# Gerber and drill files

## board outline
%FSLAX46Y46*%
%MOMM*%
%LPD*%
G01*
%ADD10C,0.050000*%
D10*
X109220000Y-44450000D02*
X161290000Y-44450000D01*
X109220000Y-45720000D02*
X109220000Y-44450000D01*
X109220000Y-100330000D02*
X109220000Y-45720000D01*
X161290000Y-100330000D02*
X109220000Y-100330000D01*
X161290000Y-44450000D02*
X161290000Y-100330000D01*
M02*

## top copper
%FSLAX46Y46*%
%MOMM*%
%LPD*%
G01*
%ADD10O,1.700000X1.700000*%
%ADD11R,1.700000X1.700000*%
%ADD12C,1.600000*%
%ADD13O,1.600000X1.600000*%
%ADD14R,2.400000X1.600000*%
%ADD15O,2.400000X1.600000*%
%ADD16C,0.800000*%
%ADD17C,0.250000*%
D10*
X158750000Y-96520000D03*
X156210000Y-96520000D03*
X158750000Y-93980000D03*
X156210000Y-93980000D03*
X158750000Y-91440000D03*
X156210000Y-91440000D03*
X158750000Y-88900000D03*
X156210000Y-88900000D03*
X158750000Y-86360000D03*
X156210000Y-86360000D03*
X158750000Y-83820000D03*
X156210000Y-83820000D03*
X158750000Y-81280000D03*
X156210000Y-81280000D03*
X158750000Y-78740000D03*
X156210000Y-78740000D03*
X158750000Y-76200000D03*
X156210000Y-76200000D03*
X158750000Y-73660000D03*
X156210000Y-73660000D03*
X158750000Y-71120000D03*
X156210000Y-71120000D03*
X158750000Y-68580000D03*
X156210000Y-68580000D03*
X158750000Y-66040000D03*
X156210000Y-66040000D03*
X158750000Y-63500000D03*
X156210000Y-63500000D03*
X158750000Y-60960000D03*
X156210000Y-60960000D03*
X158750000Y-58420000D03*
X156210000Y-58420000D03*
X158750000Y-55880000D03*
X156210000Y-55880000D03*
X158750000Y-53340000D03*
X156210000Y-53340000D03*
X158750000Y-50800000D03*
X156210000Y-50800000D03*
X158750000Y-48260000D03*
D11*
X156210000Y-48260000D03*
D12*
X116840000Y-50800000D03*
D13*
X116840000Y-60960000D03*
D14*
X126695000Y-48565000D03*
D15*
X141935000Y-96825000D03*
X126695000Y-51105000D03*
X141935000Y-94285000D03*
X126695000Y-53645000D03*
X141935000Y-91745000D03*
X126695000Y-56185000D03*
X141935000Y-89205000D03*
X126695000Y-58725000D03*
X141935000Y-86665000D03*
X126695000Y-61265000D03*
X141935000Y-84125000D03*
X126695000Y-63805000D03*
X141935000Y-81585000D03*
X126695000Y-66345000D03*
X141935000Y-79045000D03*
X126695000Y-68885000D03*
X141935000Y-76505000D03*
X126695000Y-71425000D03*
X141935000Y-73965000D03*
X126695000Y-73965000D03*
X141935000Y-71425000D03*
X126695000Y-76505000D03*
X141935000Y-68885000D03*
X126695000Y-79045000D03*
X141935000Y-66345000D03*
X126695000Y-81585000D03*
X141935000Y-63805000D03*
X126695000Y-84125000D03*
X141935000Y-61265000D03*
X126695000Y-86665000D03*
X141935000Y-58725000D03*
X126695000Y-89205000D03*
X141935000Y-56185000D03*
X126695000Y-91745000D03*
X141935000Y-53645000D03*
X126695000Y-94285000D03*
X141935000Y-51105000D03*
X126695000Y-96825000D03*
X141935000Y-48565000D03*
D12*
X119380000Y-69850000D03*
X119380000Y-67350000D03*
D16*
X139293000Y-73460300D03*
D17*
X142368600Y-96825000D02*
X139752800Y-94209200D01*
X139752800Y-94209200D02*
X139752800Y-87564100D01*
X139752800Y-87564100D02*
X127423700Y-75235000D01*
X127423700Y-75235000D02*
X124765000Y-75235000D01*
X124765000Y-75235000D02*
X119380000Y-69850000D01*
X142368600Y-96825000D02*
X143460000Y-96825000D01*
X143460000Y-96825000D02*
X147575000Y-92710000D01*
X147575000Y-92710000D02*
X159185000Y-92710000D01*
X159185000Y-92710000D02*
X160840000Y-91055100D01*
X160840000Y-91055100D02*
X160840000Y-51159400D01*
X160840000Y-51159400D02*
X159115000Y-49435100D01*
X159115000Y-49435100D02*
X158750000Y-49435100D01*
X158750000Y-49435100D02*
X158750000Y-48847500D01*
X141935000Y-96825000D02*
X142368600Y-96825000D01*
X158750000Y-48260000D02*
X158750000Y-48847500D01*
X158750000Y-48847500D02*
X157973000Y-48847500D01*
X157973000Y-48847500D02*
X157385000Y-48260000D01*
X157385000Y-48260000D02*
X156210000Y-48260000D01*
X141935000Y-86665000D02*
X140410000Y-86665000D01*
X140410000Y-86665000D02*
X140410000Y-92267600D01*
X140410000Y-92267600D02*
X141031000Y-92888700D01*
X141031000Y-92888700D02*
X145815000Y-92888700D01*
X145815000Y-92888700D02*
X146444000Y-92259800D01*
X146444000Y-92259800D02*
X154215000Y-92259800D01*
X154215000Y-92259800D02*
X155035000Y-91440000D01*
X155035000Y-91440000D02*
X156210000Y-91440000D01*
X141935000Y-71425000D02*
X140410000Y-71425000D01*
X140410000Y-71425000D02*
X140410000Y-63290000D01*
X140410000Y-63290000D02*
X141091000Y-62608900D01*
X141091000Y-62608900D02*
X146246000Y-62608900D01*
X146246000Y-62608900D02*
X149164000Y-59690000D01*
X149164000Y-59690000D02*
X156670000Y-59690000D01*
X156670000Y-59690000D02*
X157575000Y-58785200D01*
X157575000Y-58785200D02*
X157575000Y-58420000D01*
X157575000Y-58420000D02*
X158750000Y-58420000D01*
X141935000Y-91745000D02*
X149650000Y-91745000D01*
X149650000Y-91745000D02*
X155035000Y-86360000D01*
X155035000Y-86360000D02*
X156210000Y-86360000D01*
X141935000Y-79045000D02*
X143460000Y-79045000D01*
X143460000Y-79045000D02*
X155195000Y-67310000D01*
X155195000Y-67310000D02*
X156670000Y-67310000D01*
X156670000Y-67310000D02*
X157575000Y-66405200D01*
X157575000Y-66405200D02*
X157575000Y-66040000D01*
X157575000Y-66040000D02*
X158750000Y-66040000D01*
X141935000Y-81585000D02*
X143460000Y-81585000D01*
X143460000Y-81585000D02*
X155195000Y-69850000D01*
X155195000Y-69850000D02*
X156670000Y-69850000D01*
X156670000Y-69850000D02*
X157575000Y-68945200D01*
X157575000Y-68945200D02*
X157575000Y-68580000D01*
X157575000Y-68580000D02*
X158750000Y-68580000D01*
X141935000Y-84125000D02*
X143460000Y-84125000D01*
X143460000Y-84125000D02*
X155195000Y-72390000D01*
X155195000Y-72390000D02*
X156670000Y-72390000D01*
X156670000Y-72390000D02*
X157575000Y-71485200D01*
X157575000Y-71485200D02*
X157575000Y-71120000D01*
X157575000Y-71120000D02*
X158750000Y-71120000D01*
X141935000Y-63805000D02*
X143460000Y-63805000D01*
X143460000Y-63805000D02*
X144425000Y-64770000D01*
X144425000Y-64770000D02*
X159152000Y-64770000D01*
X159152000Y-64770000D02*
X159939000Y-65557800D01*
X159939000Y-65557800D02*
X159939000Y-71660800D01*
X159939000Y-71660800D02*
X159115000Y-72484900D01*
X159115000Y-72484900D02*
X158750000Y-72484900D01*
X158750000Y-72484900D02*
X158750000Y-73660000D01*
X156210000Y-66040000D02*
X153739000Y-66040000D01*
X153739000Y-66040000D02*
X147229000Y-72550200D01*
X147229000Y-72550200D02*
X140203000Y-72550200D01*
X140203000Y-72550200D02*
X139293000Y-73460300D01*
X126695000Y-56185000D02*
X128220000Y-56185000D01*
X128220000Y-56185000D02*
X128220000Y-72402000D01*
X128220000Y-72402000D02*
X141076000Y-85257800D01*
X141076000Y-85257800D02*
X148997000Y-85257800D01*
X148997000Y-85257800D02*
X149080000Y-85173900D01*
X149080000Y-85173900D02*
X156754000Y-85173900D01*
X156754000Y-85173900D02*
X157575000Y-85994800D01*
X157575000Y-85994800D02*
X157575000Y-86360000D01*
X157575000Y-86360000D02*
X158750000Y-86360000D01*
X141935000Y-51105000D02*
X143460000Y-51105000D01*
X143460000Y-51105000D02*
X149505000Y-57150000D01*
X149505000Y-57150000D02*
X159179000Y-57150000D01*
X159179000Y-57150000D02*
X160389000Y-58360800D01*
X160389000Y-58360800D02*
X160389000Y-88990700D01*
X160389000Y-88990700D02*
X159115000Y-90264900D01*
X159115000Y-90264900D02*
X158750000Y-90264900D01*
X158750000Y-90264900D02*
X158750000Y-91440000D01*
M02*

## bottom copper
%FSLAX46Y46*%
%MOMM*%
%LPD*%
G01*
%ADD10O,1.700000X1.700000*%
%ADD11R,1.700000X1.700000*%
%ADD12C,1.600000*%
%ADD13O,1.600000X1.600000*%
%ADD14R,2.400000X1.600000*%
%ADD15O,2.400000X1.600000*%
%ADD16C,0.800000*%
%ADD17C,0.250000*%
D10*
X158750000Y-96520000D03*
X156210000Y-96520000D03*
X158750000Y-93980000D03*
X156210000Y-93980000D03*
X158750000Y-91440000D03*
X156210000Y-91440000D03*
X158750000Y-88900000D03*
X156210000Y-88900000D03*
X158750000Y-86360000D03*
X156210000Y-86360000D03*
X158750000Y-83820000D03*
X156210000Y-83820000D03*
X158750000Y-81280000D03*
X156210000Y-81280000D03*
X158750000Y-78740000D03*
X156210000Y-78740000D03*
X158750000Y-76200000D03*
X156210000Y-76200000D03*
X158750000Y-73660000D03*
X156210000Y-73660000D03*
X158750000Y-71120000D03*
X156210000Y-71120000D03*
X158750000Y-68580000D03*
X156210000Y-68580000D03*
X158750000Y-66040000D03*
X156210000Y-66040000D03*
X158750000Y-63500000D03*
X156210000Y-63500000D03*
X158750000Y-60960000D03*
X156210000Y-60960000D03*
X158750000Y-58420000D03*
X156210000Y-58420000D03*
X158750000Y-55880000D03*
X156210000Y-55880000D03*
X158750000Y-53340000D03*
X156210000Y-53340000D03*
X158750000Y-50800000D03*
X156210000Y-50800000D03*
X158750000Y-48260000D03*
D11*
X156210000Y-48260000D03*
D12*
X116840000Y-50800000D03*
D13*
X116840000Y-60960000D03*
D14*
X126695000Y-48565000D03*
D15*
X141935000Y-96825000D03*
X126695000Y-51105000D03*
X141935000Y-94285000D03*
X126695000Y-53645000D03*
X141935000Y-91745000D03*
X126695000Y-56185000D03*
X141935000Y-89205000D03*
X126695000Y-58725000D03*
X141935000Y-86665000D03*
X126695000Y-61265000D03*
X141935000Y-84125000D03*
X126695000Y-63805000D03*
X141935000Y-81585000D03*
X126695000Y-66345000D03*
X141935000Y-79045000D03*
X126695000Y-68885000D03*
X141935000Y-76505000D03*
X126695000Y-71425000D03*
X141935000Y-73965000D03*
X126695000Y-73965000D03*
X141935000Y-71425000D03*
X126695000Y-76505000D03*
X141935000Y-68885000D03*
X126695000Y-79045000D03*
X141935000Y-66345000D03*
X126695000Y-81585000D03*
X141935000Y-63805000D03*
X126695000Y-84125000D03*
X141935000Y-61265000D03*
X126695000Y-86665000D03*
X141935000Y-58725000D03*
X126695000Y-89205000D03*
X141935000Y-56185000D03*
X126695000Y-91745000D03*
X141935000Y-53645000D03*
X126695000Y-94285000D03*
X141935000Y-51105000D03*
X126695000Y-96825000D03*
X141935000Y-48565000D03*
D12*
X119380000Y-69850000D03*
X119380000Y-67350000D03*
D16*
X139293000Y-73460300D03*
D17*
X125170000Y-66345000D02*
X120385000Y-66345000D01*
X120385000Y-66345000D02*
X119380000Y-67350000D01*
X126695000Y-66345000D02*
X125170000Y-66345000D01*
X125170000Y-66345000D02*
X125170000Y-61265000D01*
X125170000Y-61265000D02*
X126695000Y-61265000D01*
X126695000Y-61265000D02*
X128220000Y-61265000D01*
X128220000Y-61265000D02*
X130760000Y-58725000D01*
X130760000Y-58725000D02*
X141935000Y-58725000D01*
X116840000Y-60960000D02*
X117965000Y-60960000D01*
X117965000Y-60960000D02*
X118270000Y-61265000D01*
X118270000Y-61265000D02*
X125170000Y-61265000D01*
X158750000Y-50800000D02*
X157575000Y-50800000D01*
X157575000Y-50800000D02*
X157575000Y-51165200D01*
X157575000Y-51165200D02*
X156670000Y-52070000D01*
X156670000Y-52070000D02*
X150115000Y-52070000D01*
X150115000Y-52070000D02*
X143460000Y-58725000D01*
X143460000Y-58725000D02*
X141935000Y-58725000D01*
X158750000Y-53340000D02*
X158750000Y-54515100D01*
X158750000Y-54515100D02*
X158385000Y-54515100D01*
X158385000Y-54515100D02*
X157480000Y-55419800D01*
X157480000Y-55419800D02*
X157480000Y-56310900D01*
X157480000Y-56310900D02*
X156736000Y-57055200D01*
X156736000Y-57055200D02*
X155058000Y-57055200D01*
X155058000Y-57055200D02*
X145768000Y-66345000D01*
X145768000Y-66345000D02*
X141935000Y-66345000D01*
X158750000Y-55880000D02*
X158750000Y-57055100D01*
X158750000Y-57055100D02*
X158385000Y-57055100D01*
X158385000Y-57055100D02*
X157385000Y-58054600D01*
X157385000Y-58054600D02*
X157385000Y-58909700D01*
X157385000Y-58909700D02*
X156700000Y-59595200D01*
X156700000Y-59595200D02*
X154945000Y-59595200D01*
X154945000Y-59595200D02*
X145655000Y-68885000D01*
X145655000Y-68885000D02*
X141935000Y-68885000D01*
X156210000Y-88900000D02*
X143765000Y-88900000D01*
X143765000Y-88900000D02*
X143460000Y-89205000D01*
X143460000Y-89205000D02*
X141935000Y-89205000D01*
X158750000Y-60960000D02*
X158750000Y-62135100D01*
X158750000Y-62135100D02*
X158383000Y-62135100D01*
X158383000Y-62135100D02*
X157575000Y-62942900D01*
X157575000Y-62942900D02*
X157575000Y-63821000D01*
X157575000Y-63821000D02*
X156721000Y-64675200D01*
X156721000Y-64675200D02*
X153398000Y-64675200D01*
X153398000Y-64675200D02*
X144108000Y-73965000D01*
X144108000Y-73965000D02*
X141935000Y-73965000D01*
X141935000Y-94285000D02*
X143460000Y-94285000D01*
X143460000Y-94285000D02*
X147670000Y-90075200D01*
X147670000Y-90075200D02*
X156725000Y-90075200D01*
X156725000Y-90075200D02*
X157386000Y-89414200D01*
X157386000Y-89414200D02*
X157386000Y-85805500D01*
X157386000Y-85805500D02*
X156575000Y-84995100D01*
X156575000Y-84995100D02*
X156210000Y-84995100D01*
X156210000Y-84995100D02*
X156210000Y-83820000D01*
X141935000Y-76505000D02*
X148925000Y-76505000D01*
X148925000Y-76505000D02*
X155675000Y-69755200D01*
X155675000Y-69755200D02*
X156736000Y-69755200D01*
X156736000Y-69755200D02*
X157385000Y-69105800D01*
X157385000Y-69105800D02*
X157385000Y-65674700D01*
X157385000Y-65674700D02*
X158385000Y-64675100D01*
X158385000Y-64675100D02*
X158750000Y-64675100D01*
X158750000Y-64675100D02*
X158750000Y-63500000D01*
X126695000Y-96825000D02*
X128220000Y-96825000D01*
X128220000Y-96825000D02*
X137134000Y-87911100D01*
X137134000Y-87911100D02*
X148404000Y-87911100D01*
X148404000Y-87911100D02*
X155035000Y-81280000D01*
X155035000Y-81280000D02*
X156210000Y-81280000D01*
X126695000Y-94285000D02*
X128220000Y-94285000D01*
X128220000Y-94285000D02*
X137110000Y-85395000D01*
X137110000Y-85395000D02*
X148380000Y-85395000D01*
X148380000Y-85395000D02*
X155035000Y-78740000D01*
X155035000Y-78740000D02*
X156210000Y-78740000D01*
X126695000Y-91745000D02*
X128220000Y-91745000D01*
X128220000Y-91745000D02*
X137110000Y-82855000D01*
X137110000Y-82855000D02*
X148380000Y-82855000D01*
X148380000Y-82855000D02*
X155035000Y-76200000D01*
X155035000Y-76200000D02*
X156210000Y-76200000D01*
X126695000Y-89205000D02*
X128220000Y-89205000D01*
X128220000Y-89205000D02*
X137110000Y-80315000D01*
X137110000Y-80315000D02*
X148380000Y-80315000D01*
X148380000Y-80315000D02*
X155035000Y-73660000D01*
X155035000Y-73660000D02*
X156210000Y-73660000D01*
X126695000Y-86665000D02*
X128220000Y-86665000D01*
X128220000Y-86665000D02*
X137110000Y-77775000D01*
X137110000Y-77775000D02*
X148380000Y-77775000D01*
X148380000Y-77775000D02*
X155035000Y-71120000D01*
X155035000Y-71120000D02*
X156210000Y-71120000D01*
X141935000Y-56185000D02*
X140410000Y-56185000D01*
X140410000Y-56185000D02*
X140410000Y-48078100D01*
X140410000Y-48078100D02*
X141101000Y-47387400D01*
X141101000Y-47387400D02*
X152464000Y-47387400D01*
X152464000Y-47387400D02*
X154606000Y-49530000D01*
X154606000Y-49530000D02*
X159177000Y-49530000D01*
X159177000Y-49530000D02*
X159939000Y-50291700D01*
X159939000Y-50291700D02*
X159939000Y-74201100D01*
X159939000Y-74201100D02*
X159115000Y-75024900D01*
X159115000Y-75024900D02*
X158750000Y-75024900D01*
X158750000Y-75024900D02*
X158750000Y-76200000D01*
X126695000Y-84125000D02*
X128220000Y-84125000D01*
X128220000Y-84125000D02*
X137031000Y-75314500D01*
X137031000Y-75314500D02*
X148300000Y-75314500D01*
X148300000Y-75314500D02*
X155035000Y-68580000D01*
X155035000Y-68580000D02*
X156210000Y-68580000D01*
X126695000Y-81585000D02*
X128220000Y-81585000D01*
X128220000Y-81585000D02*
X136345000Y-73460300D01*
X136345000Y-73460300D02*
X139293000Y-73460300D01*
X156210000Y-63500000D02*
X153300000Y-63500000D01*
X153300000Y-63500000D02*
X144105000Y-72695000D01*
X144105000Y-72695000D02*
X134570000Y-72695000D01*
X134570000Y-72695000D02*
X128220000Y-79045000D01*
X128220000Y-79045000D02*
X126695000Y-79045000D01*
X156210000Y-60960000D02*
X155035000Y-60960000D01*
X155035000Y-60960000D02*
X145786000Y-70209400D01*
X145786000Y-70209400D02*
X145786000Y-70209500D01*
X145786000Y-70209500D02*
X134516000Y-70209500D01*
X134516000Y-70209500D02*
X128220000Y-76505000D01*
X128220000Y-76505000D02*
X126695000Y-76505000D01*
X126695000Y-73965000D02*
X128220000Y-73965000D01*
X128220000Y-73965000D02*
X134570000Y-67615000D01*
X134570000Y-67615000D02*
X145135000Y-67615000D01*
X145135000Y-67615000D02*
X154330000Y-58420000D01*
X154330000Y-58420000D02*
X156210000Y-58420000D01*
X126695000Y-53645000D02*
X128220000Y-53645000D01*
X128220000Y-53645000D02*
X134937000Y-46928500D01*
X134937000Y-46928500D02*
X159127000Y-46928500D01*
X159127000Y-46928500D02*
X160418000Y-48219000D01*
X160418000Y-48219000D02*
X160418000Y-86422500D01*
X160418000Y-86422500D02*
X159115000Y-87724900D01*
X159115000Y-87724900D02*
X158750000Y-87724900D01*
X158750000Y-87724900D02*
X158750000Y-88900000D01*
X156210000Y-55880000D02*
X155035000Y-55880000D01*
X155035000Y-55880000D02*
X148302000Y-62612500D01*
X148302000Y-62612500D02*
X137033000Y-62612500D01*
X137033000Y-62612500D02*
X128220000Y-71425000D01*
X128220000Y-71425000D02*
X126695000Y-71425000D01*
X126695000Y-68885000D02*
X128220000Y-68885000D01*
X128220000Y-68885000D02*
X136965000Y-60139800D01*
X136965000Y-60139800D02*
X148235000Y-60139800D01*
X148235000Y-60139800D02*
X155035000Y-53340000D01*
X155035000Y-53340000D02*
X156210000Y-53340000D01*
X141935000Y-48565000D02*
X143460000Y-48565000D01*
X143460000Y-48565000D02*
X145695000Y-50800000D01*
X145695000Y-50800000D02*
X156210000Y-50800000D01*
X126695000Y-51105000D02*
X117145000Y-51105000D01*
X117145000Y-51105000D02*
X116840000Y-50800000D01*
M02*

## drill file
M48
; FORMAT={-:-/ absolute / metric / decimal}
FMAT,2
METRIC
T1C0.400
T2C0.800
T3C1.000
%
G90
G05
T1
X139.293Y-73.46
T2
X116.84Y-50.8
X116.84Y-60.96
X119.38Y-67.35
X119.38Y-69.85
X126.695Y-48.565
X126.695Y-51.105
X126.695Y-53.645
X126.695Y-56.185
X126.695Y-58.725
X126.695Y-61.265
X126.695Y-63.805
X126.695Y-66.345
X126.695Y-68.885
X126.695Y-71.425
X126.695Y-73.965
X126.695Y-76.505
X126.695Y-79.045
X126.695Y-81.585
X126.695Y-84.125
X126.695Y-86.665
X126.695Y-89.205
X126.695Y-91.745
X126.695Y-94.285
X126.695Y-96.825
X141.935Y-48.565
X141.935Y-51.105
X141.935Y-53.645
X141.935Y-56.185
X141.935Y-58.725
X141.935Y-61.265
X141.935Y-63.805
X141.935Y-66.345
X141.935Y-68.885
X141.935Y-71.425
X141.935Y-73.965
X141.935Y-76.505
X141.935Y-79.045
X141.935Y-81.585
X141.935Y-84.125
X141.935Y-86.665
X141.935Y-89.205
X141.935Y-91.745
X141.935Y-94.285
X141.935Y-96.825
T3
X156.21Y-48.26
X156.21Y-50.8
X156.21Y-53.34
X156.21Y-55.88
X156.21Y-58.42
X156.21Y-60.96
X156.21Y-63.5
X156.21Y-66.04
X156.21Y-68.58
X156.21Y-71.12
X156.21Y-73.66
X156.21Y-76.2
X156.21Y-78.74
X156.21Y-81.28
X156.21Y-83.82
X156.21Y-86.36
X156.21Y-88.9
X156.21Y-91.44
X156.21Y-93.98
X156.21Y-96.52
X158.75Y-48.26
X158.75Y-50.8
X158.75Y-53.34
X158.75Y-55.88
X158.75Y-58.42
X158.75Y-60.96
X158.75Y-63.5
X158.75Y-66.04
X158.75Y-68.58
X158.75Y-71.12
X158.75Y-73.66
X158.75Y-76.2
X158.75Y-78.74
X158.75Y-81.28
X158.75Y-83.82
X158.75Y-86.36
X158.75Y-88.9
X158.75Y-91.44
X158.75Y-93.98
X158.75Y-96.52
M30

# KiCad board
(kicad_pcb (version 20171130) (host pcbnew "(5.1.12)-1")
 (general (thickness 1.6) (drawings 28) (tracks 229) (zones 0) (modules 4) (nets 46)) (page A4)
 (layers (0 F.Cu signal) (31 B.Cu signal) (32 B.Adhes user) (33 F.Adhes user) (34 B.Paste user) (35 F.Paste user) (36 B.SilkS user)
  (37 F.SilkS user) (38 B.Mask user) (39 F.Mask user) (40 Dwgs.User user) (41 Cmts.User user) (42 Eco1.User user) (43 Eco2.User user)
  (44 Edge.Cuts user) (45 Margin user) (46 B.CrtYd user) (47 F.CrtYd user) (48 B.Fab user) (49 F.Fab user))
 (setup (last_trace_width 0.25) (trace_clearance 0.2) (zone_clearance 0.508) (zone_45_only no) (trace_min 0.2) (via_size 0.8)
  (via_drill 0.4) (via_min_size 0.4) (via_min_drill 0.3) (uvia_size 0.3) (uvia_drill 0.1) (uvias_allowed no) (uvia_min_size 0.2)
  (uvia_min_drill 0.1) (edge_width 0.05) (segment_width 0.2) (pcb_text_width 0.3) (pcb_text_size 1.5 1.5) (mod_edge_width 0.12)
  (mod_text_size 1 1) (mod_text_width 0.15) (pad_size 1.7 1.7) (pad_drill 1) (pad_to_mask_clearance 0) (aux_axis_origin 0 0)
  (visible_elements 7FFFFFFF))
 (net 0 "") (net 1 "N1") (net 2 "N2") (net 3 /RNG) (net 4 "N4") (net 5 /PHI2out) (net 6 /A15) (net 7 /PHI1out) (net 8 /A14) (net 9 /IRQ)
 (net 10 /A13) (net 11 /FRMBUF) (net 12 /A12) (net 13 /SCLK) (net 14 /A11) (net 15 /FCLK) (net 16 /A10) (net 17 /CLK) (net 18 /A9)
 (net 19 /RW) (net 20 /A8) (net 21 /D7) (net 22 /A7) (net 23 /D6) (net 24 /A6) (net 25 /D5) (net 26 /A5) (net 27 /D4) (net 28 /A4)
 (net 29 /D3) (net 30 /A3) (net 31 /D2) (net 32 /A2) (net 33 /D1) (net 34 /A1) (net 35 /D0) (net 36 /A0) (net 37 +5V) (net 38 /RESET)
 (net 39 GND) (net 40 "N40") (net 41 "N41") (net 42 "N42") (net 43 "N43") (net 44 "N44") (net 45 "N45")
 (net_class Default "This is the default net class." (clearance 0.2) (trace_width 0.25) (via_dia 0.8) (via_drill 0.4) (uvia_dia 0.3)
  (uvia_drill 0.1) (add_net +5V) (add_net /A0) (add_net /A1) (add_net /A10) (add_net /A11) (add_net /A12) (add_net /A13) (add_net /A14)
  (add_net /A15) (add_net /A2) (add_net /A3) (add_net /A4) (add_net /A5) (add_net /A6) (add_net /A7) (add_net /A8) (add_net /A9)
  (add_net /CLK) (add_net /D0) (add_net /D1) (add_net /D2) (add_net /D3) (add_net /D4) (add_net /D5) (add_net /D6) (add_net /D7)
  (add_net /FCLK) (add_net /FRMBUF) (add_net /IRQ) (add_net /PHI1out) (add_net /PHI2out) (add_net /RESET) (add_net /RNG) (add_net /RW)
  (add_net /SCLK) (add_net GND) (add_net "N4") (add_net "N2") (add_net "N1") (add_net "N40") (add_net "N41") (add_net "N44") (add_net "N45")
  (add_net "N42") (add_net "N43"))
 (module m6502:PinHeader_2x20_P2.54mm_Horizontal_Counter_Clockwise (layer F.Cu) (at 156.21 48.26)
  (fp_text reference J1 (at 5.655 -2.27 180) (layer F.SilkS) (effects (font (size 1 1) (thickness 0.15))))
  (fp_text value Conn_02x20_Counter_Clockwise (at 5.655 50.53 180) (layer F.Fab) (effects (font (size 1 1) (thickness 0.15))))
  (pad 21 thru_hole oval (at 2.54 48.26) (size 1.7 1.7) (drill 1) (layers *.Cu *.Mask) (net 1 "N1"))
  (pad 20 thru_hole oval (at 0 48.26) (size 1.7 1.7) (drill 1) (layers *.Cu *.Mask) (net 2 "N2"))
  (pad 22 thru_hole oval (at 2.54 45.72) (size 1.7 1.7) (drill 1) (layers *.Cu *.Mask) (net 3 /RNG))
  (pad 19 thru_hole oval (at 0 45.72) (size 1.7 1.7) (drill 1) (layers *.Cu *.Mask) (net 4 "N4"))
  (pad 23 thru_hole oval (at 2.54 43.18) (size 1.7 1.7) (drill 1) (layers *.Cu *.Mask) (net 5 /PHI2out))
  (pad 18 thru_hole oval (at 0 43.18) (size 1.7 1.7) (drill 1) (layers *.Cu *.Mask) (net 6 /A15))
  (pad 24 thru_hole oval (at 2.54 40.64) (size 1.7 1.7) (drill 1) (layers *.Cu *.Mask) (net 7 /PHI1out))
  (pad 17 thru_hole oval (at 0 40.64) (size 1.7 1.7) (drill 1) (layers *.Cu *.Mask) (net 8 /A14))
  (pad 25 thru_hole oval (at 2.54 38.1) (size 1.7 1.7) (drill 1) (layers *.Cu *.Mask) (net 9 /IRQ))
  (pad 16 thru_hole oval (at 0 38.1) (size 1.7 1.7) (drill 1) (layers *.Cu *.Mask) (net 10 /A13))
  (pad 26 thru_hole oval (at 2.54 35.56) (size 1.7 1.7) (drill 1) (layers *.Cu *.Mask) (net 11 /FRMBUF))
  (pad 15 thru_hole oval (at 0 35.56) (size 1.7 1.7) (drill 1) (layers *.Cu *.Mask) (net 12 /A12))
  (pad 27 thru_hole oval (at 2.54 33.02) (size 1.7 1.7) (drill 1) (layers *.Cu *.Mask) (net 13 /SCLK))
  (pad 14 thru_hole oval (at 0 33.02) (size 1.7 1.7) (drill 1) (layers *.Cu *.Mask) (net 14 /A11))
  (pad 28 thru_hole oval (at 2.54 30.48) (size 1.7 1.7) (drill 1) (layers *.Cu *.Mask) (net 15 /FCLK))
  (pad 13 thru_hole oval (at 0 30.48) (size 1.7 1.7) (drill 1) (layers *.Cu *.Mask) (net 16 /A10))
  (pad 29 thru_hole oval (at 2.54 27.94) (size 1.7 1.7) (drill 1) (layers *.Cu *.Mask) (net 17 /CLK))
  (pad 12 thru_hole oval (at 0 27.94) (size 1.7 1.7) (drill 1) (layers *.Cu *.Mask) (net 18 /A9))
  (pad 30 thru_hole oval (at 2.54 25.4) (size 1.7 1.7) (drill 1) (layers *.Cu *.Mask) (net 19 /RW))
  (pad 11 thru_hole oval (at 0 25.4) (size 1.7 1.7) (drill 1) (layers *.Cu *.Mask) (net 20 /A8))
  (pad 31 thru_hole oval (at 2.54 22.86) (size 1.7 1.7) (drill 1) (layers *.Cu *.Mask) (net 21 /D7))
  (pad 10 thru_hole oval (at 0 22.86) (size 1.7 1.7) (drill 1) (layers *.Cu *.Mask) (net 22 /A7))
  (pad 32 thru_hole oval (at 2.54 20.32) (size 1.7 1.7) (drill 1) (layers *.Cu *.Mask) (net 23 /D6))
  (pad 9 thru_hole oval (at 0 20.32) (size 1.7 1.7) (drill 1) (layers *.Cu *.Mask) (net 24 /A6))
  (pad 33 thru_hole oval (at 2.54 17.78) (size 1.7 1.7) (drill 1) (layers *.Cu *.Mask) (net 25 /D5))
  (pad 8 thru_hole oval (at 0 17.78) (size 1.7 1.7) (drill 1) (layers *.Cu *.Mask) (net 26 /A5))
  (pad 34 thru_hole oval (at 2.54 15.24) (size 1.7 1.7) (drill 1) (layers *.Cu *.Mask) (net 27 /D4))
  (pad 7 thru_hole oval (at 0 15.24) (size 1.7 1.7) (drill 1) (layers *.Cu *.Mask) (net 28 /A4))
  (pad 35 thru_hole oval (at 2.54 12.7) (size 1.7 1.7) (drill 1) (layers *.Cu *.Mask) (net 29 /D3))
  (pad 6 thru_hole oval (at 0 12.7) (size 1.7 1.7) (drill 1) (layers *.Cu *.Mask) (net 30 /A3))
  (pad 36 thru_hole oval (at 2.54 10.16) (size 1.7 1.7) (drill 1) (layers *.Cu *.Mask) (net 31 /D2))
  (pad 5 thru_hole oval (at 0 10.16) (size 1.7 1.7) (drill 1) (layers *.Cu *.Mask) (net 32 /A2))
  (pad 37 thru_hole oval (at 2.54 7.62) (size 1.7 1.7) (drill 1) (layers *.Cu *.Mask) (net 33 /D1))
  (pad 4 thru_hole oval (at 0 7.62) (size 1.7 1.7) (drill 1) (layers *.Cu *.Mask) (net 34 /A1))
  (pad 38 thru_hole oval (at 2.54 5.08) (size 1.7 1.7) (drill 1) (layers *.Cu *.Mask) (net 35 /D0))
  (pad 3 thru_hole oval (at 0 5.08) (size 1.7 1.7) (drill 1) (layers *.Cu *.Mask) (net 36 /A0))
  (pad 39 thru_hole oval (at 2.54 2.54) (size 1.7 1.7) (drill 1) (layers *.Cu *.Mask) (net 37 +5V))
  (pad 2 thru_hole oval (at 0 2.54) (size 1.7 1.7) (drill 1) (layers *.Cu *.Mask) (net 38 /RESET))
  (pad 40 thru_hole oval (at 2.54 0) (size 1.7 1.7) (drill 1) (layers *.Cu *.Mask) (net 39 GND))
  (pad 1 thru_hole rect (at 0 0) (size 1.7 1.7) (drill 1) (layers *.Cu *.Mask) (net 39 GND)))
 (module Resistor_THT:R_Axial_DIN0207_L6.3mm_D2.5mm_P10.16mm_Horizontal (layer F.Cu) (at 116.84 50.8 270)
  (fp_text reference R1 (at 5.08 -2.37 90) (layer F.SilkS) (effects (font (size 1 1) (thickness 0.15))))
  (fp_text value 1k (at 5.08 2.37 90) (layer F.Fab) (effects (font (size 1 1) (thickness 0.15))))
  (pad 1 thru_hole circle (at 0 0 270) (size 1.6 1.6) (drill 0.8) (layers *.Cu *.Mask) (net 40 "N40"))
  (pad 2 thru_hole oval (at 10.16 0 270) (size 1.6 1.6) (drill 0.8) (layers *.Cu *.Mask) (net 37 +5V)))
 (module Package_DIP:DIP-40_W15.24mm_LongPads (layer F.Cu) (at 126.695 48.565)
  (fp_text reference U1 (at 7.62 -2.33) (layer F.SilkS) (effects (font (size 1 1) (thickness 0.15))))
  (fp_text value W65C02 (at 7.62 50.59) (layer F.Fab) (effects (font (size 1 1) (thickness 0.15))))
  (pad 1 thru_hole rect (at 0 0) (size 2.4 1.6) (drill 0.8) (layers *.Cu *.Mask) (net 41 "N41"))
  (pad 21 thru_hole oval (at 15.24 48.26) (size 2.4 1.6) (drill 0.8) (layers *.Cu *.Mask) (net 39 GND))
  (pad 2 thru_hole oval (at 0 2.54) (size 2.4 1.6) (drill 0.8) (layers *.Cu *.Mask) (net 40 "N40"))
  (pad 22 thru_hole oval (at 15.24 45.72) (size 2.4 1.6) (drill 0.8) (layers *.Cu *.Mask) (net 12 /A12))
  (pad 3 thru_hole oval (at 0 5.08) (size 2.4 1.6) (drill 0.8) (layers *.Cu *.Mask) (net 7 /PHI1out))
  (pad 23 thru_hole oval (at 15.24 43.18) (size 2.4 1.6) (drill 0.8) (layers *.Cu *.Mask) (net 10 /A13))
  (pad 4 thru_hole oval (at 0 7.62) (size 2.4 1.6) (drill 0.8) (layers *.Cu *.Mask) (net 9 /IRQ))
  (pad 24 thru_hole oval (at 15.24 40.64) (size 2.4 1.6) (drill 0.8) (layers *.Cu *.Mask) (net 8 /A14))
  (pad 5 thru_hole oval (at 0 10.16) (size 2.4 1.6) (drill 0.8) (layers *.Cu *.Mask) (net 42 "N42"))
  (pad 25 thru_hole oval (at 15.24 38.1) (size 2.4 1.6) (drill 0.8) (layers *.Cu *.Mask) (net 6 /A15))
  (pad 6 thru_hole oval (at 0 12.7) (size 2.4 1.6) (drill 0.8) (layers *.Cu *.Mask) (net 37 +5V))
  (pad 26 thru_hole oval (at 15.24 35.56) (size 2.4 1.6) (drill 0.8) (layers *.Cu *.Mask) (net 21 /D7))
  (pad 7 thru_hole oval (at 0 15.24) (size 2.4 1.6) (drill 0.8) (layers *.Cu *.Mask) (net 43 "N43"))
  (pad 27 thru_hole oval (at 15.24 33.02) (size 2.4 1.6) (drill 0.8) (layers *.Cu *.Mask) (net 23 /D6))
  (pad 8 thru_hole oval (at 0 17.78) (size 2.4 1.6) (drill 0.8) (layers *.Cu *.Mask) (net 37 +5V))
  (pad 28 thru_hole oval (at 15.24 30.48) (size 2.4 1.6) (drill 0.8) (layers *.Cu *.Mask) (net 25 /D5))
  (pad 9 thru_hole oval (at 0 20.32) (size 2.4 1.6) (drill 0.8) (layers *.Cu *.Mask) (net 36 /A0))
  (pad 29 thru_hole oval (at 15.24 27.94) (size 2.4 1.6) (drill 0.8) (layers *.Cu *.Mask) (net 27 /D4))
  (pad 10 thru_hole oval (at 0 22.86) (size 2.4 1.6) (drill 0.8) (layers *.Cu *.Mask) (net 34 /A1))
  (pad 30 thru_hole oval (at 15.24 25.4) (size 2.4 1.6) (drill 0.8) (layers *.Cu *.Mask) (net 29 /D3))
  (pad 11 thru_hole oval (at 0 25.4) (size 2.4 1.6) (drill 0.8) (layers *.Cu *.Mask) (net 32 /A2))
  (pad 31 thru_hole oval (at 15.24 22.86) (size 2.4 1.6) (drill 0.8) (layers *.Cu *.Mask) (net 31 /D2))
  (pad 12 thru_hole oval (at 0 27.94) (size 2.4 1.6) (drill 0.8) (layers *.Cu *.Mask) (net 30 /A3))
  (pad 32 thru_hole oval (at 15.24 20.32) (size 2.4 1.6) (drill 0.8) (layers *.Cu *.Mask) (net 33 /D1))
  (pad 13 thru_hole oval (at 0 30.48) (size 2.4 1.6) (drill 0.8) (layers *.Cu *.Mask) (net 28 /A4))
  (pad 33 thru_hole oval (at 15.24 17.78) (size 2.4 1.6) (drill 0.8) (layers *.Cu *.Mask) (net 35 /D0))
  (pad 14 thru_hole oval (at 0 33.02) (size 2.4 1.6) (drill 0.8) (layers *.Cu *.Mask) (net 26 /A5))
  (pad 34 thru_hole oval (at 15.24 15.24) (size 2.4 1.6) (drill 0.8) (layers *.Cu *.Mask) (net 19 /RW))
  (pad 15 thru_hole oval (at 0 35.56) (size 2.4 1.6) (drill 0.8) (layers *.Cu *.Mask) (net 24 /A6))
  (pad 35 thru_hole oval (at 15.24 12.7) (size 2.4 1.6) (drill 0.8) (layers *.Cu *.Mask) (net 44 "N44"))
  (pad 16 thru_hole oval (at 0 38.1) (size 2.4 1.6) (drill 0.8) (layers *.Cu *.Mask) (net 22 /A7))
  (pad 36 thru_hole oval (at 15.24 10.16) (size 2.4 1.6) (drill 0.8) (layers *.Cu *.Mask) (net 37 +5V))
  (pad 17 thru_hole oval (at 0 40.64) (size 2.4 1.6) (drill 0.8) (layers *.Cu *.Mask) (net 20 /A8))
  (pad 37 thru_hole oval (at 15.24 7.62) (size 2.4 1.6) (drill 0.8) (layers *.Cu *.Mask) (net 17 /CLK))
  (pad 18 thru_hole oval (at 0 43.18) (size 2.4 1.6) (drill 0.8) (layers *.Cu *.Mask) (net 18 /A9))
  (pad 38 thru_hole oval (at 15.24 5.08) (size 2.4 1.6) (drill 0.8) (layers *.Cu *.Mask) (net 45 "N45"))
  (pad 19 thru_hole oval (at 0 45.72) (size 2.4 1.6) (drill 0.8) (layers *.Cu *.Mask) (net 16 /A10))
  (pad 39 thru_hole oval (at 15.24 2.54) (size 2.4 1.6) (drill 0.8) (layers *.Cu *.Mask) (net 5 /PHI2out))
  (pad 20 thru_hole oval (at 0 48.26) (size 2.4 1.6) (drill 0.8) (layers *.Cu *.Mask) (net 14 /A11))
  (pad 40 thru_hole oval (at 15.24 0) (size 2.4 1.6) (drill 0.8) (layers *.Cu *.Mask) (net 38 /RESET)))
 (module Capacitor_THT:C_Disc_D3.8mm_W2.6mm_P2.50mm (layer F.Cu) (at 119.38 69.85 90)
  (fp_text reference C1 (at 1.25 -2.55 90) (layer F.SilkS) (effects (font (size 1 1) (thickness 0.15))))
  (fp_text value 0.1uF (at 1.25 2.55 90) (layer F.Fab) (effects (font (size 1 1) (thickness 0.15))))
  (pad 1 thru_hole circle (at 0 0 90) (size 1.6 1.6) (drill 0.8) (layers *.Cu *.Mask) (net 39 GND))
  (pad 2 thru_hole circle (at 2.5 0 90) (size 1.6 1.6) (drill 0.8) (layers *.Cu *.Mask) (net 37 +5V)))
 (gr_line (start 109.22 44.45) (end 161.29 44.45) (layer Edge.Cuts) (width 0.05))
 (gr_line (start 109.22 45.72) (end 109.22 44.45) (layer Edge.Cuts) (width 0.05))
 (gr_line (start 109.22 100.33) (end 109.22 45.72) (layer Edge.Cuts) (width 0.05))
 (gr_line (start 161.29 100.33) (end 109.22 100.33) (layer Edge.Cuts) (width 0.05))
 (gr_line (start 161.29 44.45) (end 161.29 100.33) (layer Edge.Cuts) (width 0.05))
 (segment (start 142.3686 96.825) (end 139.7528 94.2092) (width 0.25) (layer F.Cu) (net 39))
 (segment (start 139.7528 94.2092) (end 139.7528 87.5641) (width 0.25) (layer F.Cu) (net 39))
 (segment (start 139.7528 87.5641) (end 127.4237 75.235) (width 0.25) (layer F.Cu) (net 39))
 (segment (start 127.4237 75.235) (end 124.765 75.235) (width 0.25) (layer F.Cu) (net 39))
 (segment (start 124.765 75.235) (end 119.38 69.85) (width 0.25) (layer F.Cu) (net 39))
 (segment (start 142.3686 96.825) (end 143.46 96.825) (width 0.25) (layer F.Cu) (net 39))
 (segment (start 143.46 96.825) (end 147.575 92.71) (width 0.25) (layer F.Cu) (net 39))
 (segment (start 147.575 92.71) (end 159.185 92.71) (width 0.25) (layer F.Cu) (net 39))
 (segment (start 159.185 92.71) (end 160.84 91.0551) (width 0.25) (layer F.Cu) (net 39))
 (segment (start 160.84 91.0551) (end 160.84 51.1594) (width 0.25) (layer F.Cu) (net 39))
 (segment (start 160.84 51.1594) (end 159.115 49.4351) (width 0.25) (layer F.Cu) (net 39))
 (segment (start 159.115 49.4351) (end 158.75 49.4351) (width 0.25) (layer F.Cu) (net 39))
 (segment (start 158.75 49.4351) (end 158.75 48.8475) (width 0.25) (layer F.Cu) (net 39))
 (segment (start 141.935 96.825) (end 142.3686 96.825) (width 0.25) (layer F.Cu) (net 39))
 (segment (start 158.75 48.26) (end 158.75 48.8475) (width 0.25) (layer F.Cu) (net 39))
 (segment (start 158.75 48.8475) (end 157.973 48.8475) (width 0.25) (layer F.Cu) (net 39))
 (segment (start 157.973 48.8475) (end 157.385 48.26) (width 0.25) (layer F.Cu) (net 39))
 (segment (start 157.385 48.26) (end 156.21 48.26) (width 0.25) (layer F.Cu) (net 39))
 (segment (start 125.17 66.345) (end 120.385 66.345) (width 0.25) (layer B.Cu) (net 37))
 (segment (start 120.385 66.345) (end 119.38 67.35) (width 0.25) (layer B.Cu) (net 37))
 (segment (start 126.695 66.345) (end 125.17 66.345) (width 0.25) (layer B.Cu) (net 37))
 (segment (start 125.17 66.345) (end 125.17 61.265) (width 0.25) (layer B.Cu) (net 37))
 (segment (start 125.17 61.265) (end 126.695 61.265) (width 0.25) (layer B.Cu) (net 37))
 (segment (start 126.695 61.265) (end 128.22 61.265) (width 0.25) (layer B.Cu) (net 37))
 (segment (start 128.22 61.265) (end 130.76 58.725) (width 0.25) (layer B.Cu) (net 37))
 (segment (start 130.76 58.725) (end 141.935 58.725) (width 0.25) (layer B.Cu) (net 37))
 (segment (start 116.84 60.96) (end 117.965 60.96) (width 0.25) (layer B.Cu) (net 37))
 (segment (start 117.965 60.96) (end 118.27 61.265) (width 0.25) (layer B.Cu) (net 37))
 (segment (start 118.27 61.265) (end 125.17 61.265) (width 0.25) (layer B.Cu) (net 37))
 (segment (start 158.75 50.8) (end 157.575 50.8) (width 0.25) (layer B.Cu) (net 37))
 (segment (start 157.575 50.8) (end 157.575 51.1652) (width 0.25) (layer B.Cu) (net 37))
 (segment (start 157.575 51.1652) (end 156.67 52.07) (width 0.25) (layer B.Cu) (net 37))
 (segment (start 156.67 52.07) (end 150.115 52.07) (width 0.25) (layer B.Cu) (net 37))
 (segment (start 150.115 52.07) (end 143.46 58.725) (width 0.25) (layer B.Cu) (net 37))
 (segment (start 143.46 58.725) (end 141.935 58.725) (width 0.25) (layer B.Cu) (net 37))
 (segment (start 158.75 53.34) (end 158.75 54.5151) (width 0.25) (layer B.Cu) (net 35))
 (segment (start 158.75 54.5151) (end 158.385 54.5151) (width 0.25) (layer B.Cu) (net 35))
 (segment (start 158.385 54.5151) (end 157.48 55.4198) (width 0.25) (layer B.Cu) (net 35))
 (segment (start 157.48 55.4198) (end 157.48 56.3109) (width 0.25) (layer B.Cu) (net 35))
 (segment (start 157.48 56.3109) (end 156.736 57.0552) (width 0.25) (layer B.Cu) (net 35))
 (segment (start 156.736 57.0552) (end 155.058 57.0552) (width 0.25) (layer B.Cu) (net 35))
 (segment (start 155.058 57.0552) (end 145.768 66.345) (width 0.25) (layer B.Cu) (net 35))
 (segment (start 145.768 66.345) (end 141.935 66.345) (width 0.25) (layer B.Cu) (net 35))
 (segment (start 141.935 86.665) (end 140.41 86.665) (width 0.25) (layer F.Cu) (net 6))
 (segment (start 140.41 86.665) (end 140.41 92.2676) (width 0.25) (layer F.Cu) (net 6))
 (segment (start 140.41 92.2676) (end 141.031 92.8887) (width 0.25) (layer F.Cu) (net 6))
 (segment (start 141.031 92.8887) (end 145.815 92.8887) (width 0.25) (layer F.Cu) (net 6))
 (segment (start 145.815 92.8887) (end 146.444 92.2598) (width 0.25) (layer F.Cu) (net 6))
 (segment (start 146.444 92.2598) (end 154.215 92.2598) (width 0.25) (layer F.Cu) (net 6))
 (segment (start 154.215 92.2598) (end 155.035 91.44) (width 0.25) (layer F.Cu) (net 6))
 (segment (start 155.035 91.44) (end 156.21 91.44) (width 0.25) (layer F.Cu) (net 6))
 (segment (start 158.75 55.88) (end 158.75 57.0551) (width 0.25) (layer B.Cu) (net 33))
 (segment (start 158.75 57.0551) (end 158.385 57.0551) (width 0.25) (layer B.Cu) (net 33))
 (segment (start 158.385 57.0551) (end 157.385 58.0546) (width 0.25) (layer B.Cu) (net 33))
 (segment (start 157.385 58.0546) (end 157.385 58.9097) (width 0.25) (layer B.Cu) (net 33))
 (segment (start 157.385 58.9097) (end 156.7 59.5952) (width 0.25) (layer B.Cu) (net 33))
 (segment (start 156.7 59.5952) (end 154.945 59.5952) (width 0.25) (layer B.Cu) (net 33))
 (segment (start 154.945 59.5952) (end 145.655 68.885) (width 0.25) (layer B.Cu) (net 33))
 (segment (start 145.655 68.885) (end 141.935 68.885) (width 0.25) (layer B.Cu) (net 33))
 (segment (start 156.21 88.9) (end 143.765 88.9) (width 0.25) (layer B.Cu) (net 8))
 (segment (start 143.765 88.9) (end 143.46 89.205) (width 0.25) (layer B.Cu) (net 8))
 (segment (start 143.46 89.205) (end 141.935 89.205) (width 0.25) (layer B.Cu) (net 8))
 (segment (start 141.935 71.425) (end 140.41 71.425) (width 0.25) (layer F.Cu) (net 31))
 (segment (start 140.41 71.425) (end 140.41 63.29) (width 0.25) (layer F.Cu) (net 31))
 (segment (start 140.41 63.29) (end 141.091 62.6089) (width 0.25) (layer F.Cu) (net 31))
 (segment (start 141.091 62.6089) (end 146.246 62.6089) (width 0.25) (layer F.Cu) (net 31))
 (segment (start 146.246 62.6089) (end 149.164 59.69) (width 0.25) (layer F.Cu) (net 31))
 (segment (start 149.164 59.69) (end 156.67 59.69) (width 0.25) (layer F.Cu) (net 31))
 (segment (start 156.67 59.69) (end 157.575 58.7852) (width 0.25) (layer F.Cu) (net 31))
 (segment (start 157.575 58.7852) (end 157.575 58.42) (width 0.25) (layer F.Cu) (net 31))
 (segment (start 157.575 58.42) (end 158.75 58.42) (width 0.25) (layer F.Cu) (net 31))
 (segment (start 141.935 91.745) (end 149.65 91.745) (width 0.25) (layer F.Cu) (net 10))
 (segment (start 149.65 91.745) (end 155.035 86.36) (width 0.25) (layer F.Cu) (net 10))
 (segment (start 155.035 86.36) (end 156.21 86.36) (width 0.25) (layer F.Cu) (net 10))
 (segment (start 158.75 60.96) (end 158.75 62.1351) (width 0.25) (layer B.Cu) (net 29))
 (segment (start 158.75 62.1351) (end 158.383 62.1351) (width 0.25) (layer B.Cu) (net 29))
 (segment (start 158.383 62.1351) (end 157.575 62.9429) (width 0.25) (layer B.Cu) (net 29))
 (segment (start 157.575 62.9429) (end 157.575 63.821) (width 0.25) (layer B.Cu) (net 29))
 (segment (start 157.575 63.821) (end 156.721 64.6752) (width 0.25) (layer B.Cu) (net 29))
 (segment (start 156.721 64.6752) (end 153.398 64.6752) (width 0.25) (layer B.Cu) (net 29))
 (segment (start 153.398 64.6752) (end 144.108 73.965) (width 0.25) (layer B.Cu) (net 29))
 (segment (start 144.108 73.965) (end 141.935 73.965) (width 0.25) (layer B.Cu) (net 29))
 (segment (start 141.935 94.285) (end 143.46 94.285) (width 0.25) (layer B.Cu) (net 12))
 (segment (start 143.46 94.285) (end 147.67 90.0752) (width 0.25) (layer B.Cu) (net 12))
 (segment (start 147.67 90.0752) (end 156.725 90.0752) (width 0.25) (layer B.Cu) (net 12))
 (segment (start 156.725 90.0752) (end 157.386 89.4142) (width 0.25) (layer B.Cu) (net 12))
 (segment (start 157.386 89.4142) (end 157.386 85.8055) (width 0.25) (layer B.Cu) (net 12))
 (segment (start 157.386 85.8055) (end 156.575 84.9951) (width 0.25) (layer B.Cu) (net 12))
 (segment (start 156.575 84.9951) (end 156.21 84.9951) (width 0.25) (layer B.Cu) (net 12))
 (segment (start 156.21 84.9951) (end 156.21 83.82) (width 0.25) (layer B.Cu) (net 12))
 (segment (start 141.935 76.505) (end 148.925 76.505) (width 0.25) (layer B.Cu) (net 27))
 (segment (start 148.925 76.505) (end 155.675 69.7552) (width 0.25) (layer B.Cu) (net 27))
 (segment (start 155.675 69.7552) (end 156.736 69.7552) (width 0.25) (layer B.Cu) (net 27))
 (segment (start 156.736 69.7552) (end 157.385 69.1058) (width 0.25) (layer B.Cu) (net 27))
 (segment (start 157.385 69.1058) (end 157.385 65.6747) (width 0.25) (layer B.Cu) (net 27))
 (segment (start 157.385 65.6747) (end 158.385 64.6751) (width 0.25) (layer B.Cu) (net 27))
 (segment (start 158.385 64.6751) (end 158.75 64.6751) (width 0.25) (layer B.Cu) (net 27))
 (segment (start 158.75 64.6751) (end 158.75 63.5) (width 0.25) (layer B.Cu) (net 27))
 (segment (start 126.695 96.825) (end 128.22 96.825) (width 0.25) (layer B.Cu) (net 14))
 (segment (start 128.22 96.825) (end 137.134 87.9111) (width 0.25) (layer B.Cu) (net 14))
 (segment (start 137.134 87.9111) (end 148.404 87.9111) (width 0.25) (layer B.Cu) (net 14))
 (segment (start 148.404 87.9111) (end 155.035 81.28) (width 0.25) (layer B.Cu) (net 14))
 (segment (start 155.035 81.28) (end 156.21 81.28) (width 0.25) (layer B.Cu) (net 14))
 (segment (start 141.935 79.045) (end 143.46 79.045) (width 0.25) (layer F.Cu) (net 25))
 (segment (start 143.46 79.045) (end 155.195 67.31) (width 0.25) (layer F.Cu) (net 25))
 (segment (start 155.195 67.31) (end 156.67 67.31) (width 0.25) (layer F.Cu) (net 25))
 (segment (start 156.67 67.31) (end 157.575 66.4052) (width 0.25) (layer F.Cu) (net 25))
 (segment (start 157.575 66.4052) (end 157.575 66.04) (width 0.25) (layer F.Cu) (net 25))
 (segment (start 157.575 66.04) (end 158.75 66.04) (width 0.25) (layer F.Cu) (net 25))
 (segment (start 126.695 94.285) (end 128.22 94.285) (width 0.25) (layer B.Cu) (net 16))
 (segment (start 128.22 94.285) (end 137.11 85.395) (width 0.25) (layer B.Cu) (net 16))
 (segment (start 137.11 85.395) (end 148.38 85.395) (width 0.25) (layer B.Cu) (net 16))
 (segment (start 148.38 85.395) (end 155.035 78.74) (width 0.25) (layer B.Cu) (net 16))
 (segment (start 155.035 78.74) (end 156.21 78.74) (width 0.25) (layer B.Cu) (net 16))
 (segment (start 141.935 81.585) (end 143.46 81.585) (width 0.25) (layer F.Cu) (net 23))
 (segment (start 143.46 81.585) (end 155.195 69.85) (width 0.25) (layer F.Cu) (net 23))
 (segment (start 155.195 69.85) (end 156.67 69.85) (width 0.25) (layer F.Cu) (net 23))
 (segment (start 156.67 69.85) (end 157.575 68.9452) (width 0.25) (layer F.Cu) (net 23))
 (segment (start 157.575 68.9452) (end 157.575 68.58) (width 0.25) (layer F.Cu) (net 23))
 (segment (start 157.575 68.58) (end 158.75 68.58) (width 0.25) (layer F.Cu) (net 23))
 (segment (start 126.695 91.745) (end 128.22 91.745) (width 0.25) (layer B.Cu) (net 18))
 (segment (start 128.22 91.745) (end 137.11 82.855) (width 0.25) (layer B.Cu) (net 18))
 (segment (start 137.11 82.855) (end 148.38 82.855) (width 0.25) (layer B.Cu) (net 18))
 (segment (start 148.38 82.855) (end 155.035 76.2) (width 0.25) (layer B.Cu) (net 18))
 (segment (start 155.035 76.2) (end 156.21 76.2) (width 0.25) (layer B.Cu) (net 18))
 (segment (start 141.935 84.125) (end 143.46 84.125) (width 0.25) (layer F.Cu) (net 21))
 (segment (start 143.46 84.125) (end 155.195 72.39) (width 0.25) (layer F.Cu) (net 21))
 (segment (start 155.195 72.39) (end 156.67 72.39) (width 0.25) (layer F.Cu) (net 21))
 (segment (start 156.67 72.39) (end 157.575 71.4852) (width 0.25) (layer F.Cu) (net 21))
 (segment (start 157.575 71.4852) (end 157.575 71.12) (width 0.25) (layer F.Cu) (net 21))
 (segment (start 157.575 71.12) (end 158.75 71.12) (width 0.25) (layer F.Cu) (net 21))
 (segment (start 126.695 89.205) (end 128.22 89.205) (width 0.25) (layer B.Cu) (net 20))
 (segment (start 128.22 89.205) (end 137.11 80.315) (width 0.25) (layer B.Cu) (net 20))
 (segment (start 137.11 80.315) (end 148.38 80.315) (width 0.25) (layer B.Cu) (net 20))
 (segment (start 148.38 80.315) (end 155.035 73.66) (width 0.25) (layer B.Cu) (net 20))
 (segment (start 155.035 73.66) (end 156.21 73.66) (width 0.25) (layer B.Cu) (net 20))
 (segment (start 141.935 63.805) (end 143.46 63.805) (width 0.25) (layer F.Cu) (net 19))
 (segment (start 143.46 63.805) (end 144.425 64.77) (width 0.25) (layer F.Cu) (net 19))
 (segment (start 144.425 64.77) (end 159.152 64.77) (width 0.25) (layer F.Cu) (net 19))
 (segment (start 159.152 64.77) (end 159.939 65.5578) (width 0.25) (layer F.Cu) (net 19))
 (segment (start 159.939 65.5578) (end 159.939 71.6608) (width 0.25) (layer F.Cu) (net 19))
 (segment (start 159.939 71.6608) (end 159.115 72.4849) (width 0.25) (layer F.Cu) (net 19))
 (segment (start 159.115 72.4849) (end 158.75 72.4849) (width 0.25) (layer F.Cu) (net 19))
 (segment (start 158.75 72.4849) (end 158.75 73.66) (width 0.25) (layer F.Cu) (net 19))
 (segment (start 126.695 86.665) (end 128.22 86.665) (width 0.25) (layer B.Cu) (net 22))
 (segment (start 128.22 86.665) (end 137.11 77.775) (width 0.25) (layer B.Cu) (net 22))
 (segment (start 137.11 77.775) (end 148.38 77.775) (width 0.25) (layer B.Cu) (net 22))
 (segment (start 148.38 77.775) (end 155.035 71.12) (width 0.25) (layer B.Cu) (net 22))
 (segment (start 155.035 71.12) (end 156.21 71.12) (width 0.25) (layer B.Cu) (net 22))
 (segment (start 141.935 56.185) (end 140.41 56.185) (width 0.25) (layer B.Cu) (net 17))
 (segment (start 140.41 56.185) (end 140.41 48.0781) (width 0.25) (layer B.Cu) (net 17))
 (segment (start 140.41 48.0781) (end 141.101 47.3874) (width 0.25) (layer B.Cu) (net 17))
 (segment (start 141.101 47.3874) (end 152.464 47.3874) (width 0.25) (layer B.Cu) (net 17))
 (segment (start 152.464 47.3874) (end 154.606 49.53) (width 0.25) (layer B.Cu) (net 17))
 (segment (start 154.606 49.53) (end 159.177 49.53) (width 0.25) (layer B.Cu) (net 17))
 (segment (start 159.177 49.53) (end 159.939 50.2917) (width 0.25) (layer B.Cu) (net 17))
 (segment (start 159.939 50.2917) (end 159.939 74.2011) (width 0.25) (layer B.Cu) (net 17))
 (segment (start 159.939 74.2011) (end 159.115 75.0249) (width 0.25) (layer B.Cu) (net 17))
 (segment (start 159.115 75.0249) (end 158.75 75.0249) (width 0.25) (layer B.Cu) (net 17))
 (segment (start 158.75 75.0249) (end 158.75 76.2) (width 0.25) (layer B.Cu) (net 17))
 (segment (start 126.695 84.125) (end 128.22 84.125) (width 0.25) (layer B.Cu) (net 24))
 (segment (start 128.22 84.125) (end 137.031 75.3145) (width 0.25) (layer B.Cu) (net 24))
 (segment (start 137.031 75.3145) (end 148.3 75.3145) (width 0.25) (layer B.Cu) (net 24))
 (segment (start 148.3 75.3145) (end 155.035 68.58) (width 0.25) (layer B.Cu) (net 24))
 (segment (start 155.035 68.58) (end 156.21 68.58) (width 0.25) (layer B.Cu) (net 24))
 (segment (start 126.695 81.585) (end 128.22 81.585) (width 0.25) (layer B.Cu) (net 26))
 (segment (start 128.22 81.585) (end 136.345 73.4603) (width 0.25) (layer B.Cu) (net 26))
 (segment (start 136.345 73.4603) (end 139.293 73.4603) (width 0.25) (layer B.Cu) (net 26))
 (segment (start 156.21 66.04) (end 153.739 66.04) (width 0.25) (layer F.Cu) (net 26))
 (segment (start 153.739 66.04) (end 147.229 72.5502) (width 0.25) (layer F.Cu) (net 26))
 (segment (start 147.229 72.5502) (end 140.203 72.5502) (width 0.25) (layer F.Cu) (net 26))
 (segment (start 140.203 72.5502) (end 139.293 73.4603) (width 0.25) (layer F.Cu) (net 26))
 (via (at 139.293 73.4603) (size 0.8) (layers F.Cu B.Cu) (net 26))
 (segment (start 156.21 63.5) (end 153.3 63.5) (width 0.25) (layer B.Cu) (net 28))
 (segment (start 153.3 63.5) (end 144.105 72.695) (width 0.25) (layer B.Cu) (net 28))
 (segment (start 144.105 72.695) (end 134.57 72.695) (width 0.25) (layer B.Cu) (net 28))
 (segment (start 134.57 72.695) (end 128.22 79.045) (width 0.25) (layer B.Cu) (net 28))
 (segment (start 128.22 79.045) (end 126.695 79.045) (width 0.25) (layer B.Cu) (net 28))
 (segment (start 156.21 60.96) (end 155.035 60.96) (width 0.25) (layer B.Cu) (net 30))
 (segment (start 155.035 60.96) (end 145.786 70.2094) (width 0.25) (layer B.Cu) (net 30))
 (segment (start 145.786 70.2094) (end 145.786 70.2095) (width 0.25) (layer B.Cu) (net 30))
 (segment (start 145.786 70.2095) (end 134.516 70.2095) (width 0.25) (layer B.Cu) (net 30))
 (segment (start 134.516 70.2095) (end 128.22 76.505) (width 0.25) (layer B.Cu) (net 30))
 (segment (start 128.22 76.505) (end 126.695 76.505) (width 0.25) (layer B.Cu) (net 30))
 (segment (start 126.695 56.185) (end 128.22 56.185) (width 0.25) (layer F.Cu) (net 9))
 (segment (start 128.22 56.185) (end 128.22 72.402) (width 0.25) (layer F.Cu) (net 9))
 (segment (start 128.22 72.402) (end 141.076 85.2578) (width 0.25) (layer F.Cu) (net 9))
 (segment (start 141.076 85.2578) (end 148.997 85.2578) (width 0.25) (layer F.Cu) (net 9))
 (segment (start 148.997 85.2578) (end 149.08 85.1739) (width 0.25) (layer F.Cu) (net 9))
 (segment (start 149.08 85.1739) (end 156.754 85.1739) (width 0.25) (layer F.Cu) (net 9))
 (segment (start 156.754 85.1739) (end 157.575 85.9948) (width 0.25) (layer F.Cu) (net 9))
 (segment (start 157.575 85.9948) (end 157.575 86.36) (width 0.25) (layer F.Cu) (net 9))
 (segment (start 157.575 86.36) (end 158.75 86.36) (width 0.25) (layer F.Cu) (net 9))
 (segment (start 126.695 73.965) (end 128.22 73.965) (width 0.25) (layer B.Cu) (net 32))
 (segment (start 128.22 73.965) (end 134.57 67.615) (width 0.25) (layer B.Cu) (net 32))
 (segment (start 134.57 67.615) (end 145.135 67.615) (width 0.25) (layer B.Cu) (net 32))
 (segment (start 145.135 67.615) (end 154.33 58.42) (width 0.25) (layer B.Cu) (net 32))
 (segment (start 154.33 58.42) (end 156.21 58.42) (width 0.25) (layer B.Cu) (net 32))
 (segment (start 126.695 53.645) (end 128.22 53.645) (width 0.25) (layer B.Cu) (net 7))
 (segment (start 128.22 53.645) (end 134.937 46.9285) (width 0.25) (layer B.Cu) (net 7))
 (segment (start 134.937 46.9285) (end 159.127 46.9285) (width 0.25) (layer B.Cu) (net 7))
 (segment (start 159.127 46.9285) (end 160.418 48.219) (width 0.25) (layer B.Cu) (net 7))
 (segment (start 160.418 48.219) (end 160.418 86.4225) (width 0.25) (layer B.Cu) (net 7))
 (segment (start 160.418 86.4225) (end 159.115 87.7249) (width 0.25) (layer B.Cu) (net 7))
 (segment (start 159.115 87.7249) (end 158.75 87.7249) (width 0.25) (layer B.Cu) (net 7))
 (segment (start 158.75 87.7249) (end 158.75 88.9) (width 0.25) (layer B.Cu) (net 7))
 (segment (start 156.21 55.88) (end 155.035 55.88) (width 0.25) (layer B.Cu) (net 34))
 (segment (start 155.035 55.88) (end 148.302 62.6125) (width 0.25) (layer B.Cu) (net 34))
 (segment (start 148.302 62.6125) (end 137.033 62.6125) (width 0.25) (layer B.Cu) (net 34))
 (segment (start 137.033 62.6125) (end 128.22 71.425) (width 0.25) (layer B.Cu) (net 34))
 (segment (start 128.22 71.425) (end 126.695 71.425) (width 0.25) (layer B.Cu) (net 34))
 (segment (start 141.935 51.105) (end 143.46 51.105) (width 0.25) (layer F.Cu) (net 5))
 (segment (start 143.46 51.105) (end 149.505 57.15) (width 0.25) (layer F.Cu) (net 5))
 (segment (start 149.505 57.15) (end 159.179 57.15) (width 0.25) (layer F.Cu) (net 5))
 (segment (start 159.179 57.15) (end 160.389 58.3608) (width 0.25) (layer F.Cu) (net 5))
 (segment (start 160.389 58.3608) (end 160.389 88.9907) (width 0.25) (layer F.Cu) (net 5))
 (segment (start 160.389 88.9907) (end 159.115 90.2649) (width 0.25) (layer F.Cu) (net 5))
 (segment (start 159.115 90.2649) (end 158.75 90.2649) (width 0.25) (layer F.Cu) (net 5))
 (segment (start 158.75 90.2649) (end 158.75 91.44) (width 0.25) (layer F.Cu) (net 5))
 (segment (start 126.695 68.885) (end 128.22 68.885) (width 0.25) (layer B.Cu) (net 36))
 (segment (start 128.22 68.885) (end 136.965 60.1398) (width 0.25) (layer B.Cu) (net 36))
 (segment (start 136.965 60.1398) (end 148.235 60.1398) (width 0.25) (layer B.Cu) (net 36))
 (segment (start 148.235 60.1398) (end 155.035 53.34) (width 0.25) (layer B.Cu) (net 36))
 (segment (start 155.035 53.34) (end 156.21 53.34) (width 0.25) (layer B.Cu) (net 36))
 (segment (start 141.935 48.565) (end 143.46 48.565) (width 0.25) (layer B.Cu) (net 38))
 (segment (start 143.46 48.565) (end 145.695 50.8) (width 0.25) (layer B.Cu) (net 38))
 (segment (start 145.695 50.8) (end 156.21 50.8) (width 0.25) (layer B.Cu) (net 38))
 (segment (start 126.695 51.105) (end 117.145 51.105) (width 0.25) (layer B.Cu) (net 40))
 (segment (start 117.145 51.105) (end 116.84 50.8) (width 0.25) (layer B.Cu) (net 40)))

